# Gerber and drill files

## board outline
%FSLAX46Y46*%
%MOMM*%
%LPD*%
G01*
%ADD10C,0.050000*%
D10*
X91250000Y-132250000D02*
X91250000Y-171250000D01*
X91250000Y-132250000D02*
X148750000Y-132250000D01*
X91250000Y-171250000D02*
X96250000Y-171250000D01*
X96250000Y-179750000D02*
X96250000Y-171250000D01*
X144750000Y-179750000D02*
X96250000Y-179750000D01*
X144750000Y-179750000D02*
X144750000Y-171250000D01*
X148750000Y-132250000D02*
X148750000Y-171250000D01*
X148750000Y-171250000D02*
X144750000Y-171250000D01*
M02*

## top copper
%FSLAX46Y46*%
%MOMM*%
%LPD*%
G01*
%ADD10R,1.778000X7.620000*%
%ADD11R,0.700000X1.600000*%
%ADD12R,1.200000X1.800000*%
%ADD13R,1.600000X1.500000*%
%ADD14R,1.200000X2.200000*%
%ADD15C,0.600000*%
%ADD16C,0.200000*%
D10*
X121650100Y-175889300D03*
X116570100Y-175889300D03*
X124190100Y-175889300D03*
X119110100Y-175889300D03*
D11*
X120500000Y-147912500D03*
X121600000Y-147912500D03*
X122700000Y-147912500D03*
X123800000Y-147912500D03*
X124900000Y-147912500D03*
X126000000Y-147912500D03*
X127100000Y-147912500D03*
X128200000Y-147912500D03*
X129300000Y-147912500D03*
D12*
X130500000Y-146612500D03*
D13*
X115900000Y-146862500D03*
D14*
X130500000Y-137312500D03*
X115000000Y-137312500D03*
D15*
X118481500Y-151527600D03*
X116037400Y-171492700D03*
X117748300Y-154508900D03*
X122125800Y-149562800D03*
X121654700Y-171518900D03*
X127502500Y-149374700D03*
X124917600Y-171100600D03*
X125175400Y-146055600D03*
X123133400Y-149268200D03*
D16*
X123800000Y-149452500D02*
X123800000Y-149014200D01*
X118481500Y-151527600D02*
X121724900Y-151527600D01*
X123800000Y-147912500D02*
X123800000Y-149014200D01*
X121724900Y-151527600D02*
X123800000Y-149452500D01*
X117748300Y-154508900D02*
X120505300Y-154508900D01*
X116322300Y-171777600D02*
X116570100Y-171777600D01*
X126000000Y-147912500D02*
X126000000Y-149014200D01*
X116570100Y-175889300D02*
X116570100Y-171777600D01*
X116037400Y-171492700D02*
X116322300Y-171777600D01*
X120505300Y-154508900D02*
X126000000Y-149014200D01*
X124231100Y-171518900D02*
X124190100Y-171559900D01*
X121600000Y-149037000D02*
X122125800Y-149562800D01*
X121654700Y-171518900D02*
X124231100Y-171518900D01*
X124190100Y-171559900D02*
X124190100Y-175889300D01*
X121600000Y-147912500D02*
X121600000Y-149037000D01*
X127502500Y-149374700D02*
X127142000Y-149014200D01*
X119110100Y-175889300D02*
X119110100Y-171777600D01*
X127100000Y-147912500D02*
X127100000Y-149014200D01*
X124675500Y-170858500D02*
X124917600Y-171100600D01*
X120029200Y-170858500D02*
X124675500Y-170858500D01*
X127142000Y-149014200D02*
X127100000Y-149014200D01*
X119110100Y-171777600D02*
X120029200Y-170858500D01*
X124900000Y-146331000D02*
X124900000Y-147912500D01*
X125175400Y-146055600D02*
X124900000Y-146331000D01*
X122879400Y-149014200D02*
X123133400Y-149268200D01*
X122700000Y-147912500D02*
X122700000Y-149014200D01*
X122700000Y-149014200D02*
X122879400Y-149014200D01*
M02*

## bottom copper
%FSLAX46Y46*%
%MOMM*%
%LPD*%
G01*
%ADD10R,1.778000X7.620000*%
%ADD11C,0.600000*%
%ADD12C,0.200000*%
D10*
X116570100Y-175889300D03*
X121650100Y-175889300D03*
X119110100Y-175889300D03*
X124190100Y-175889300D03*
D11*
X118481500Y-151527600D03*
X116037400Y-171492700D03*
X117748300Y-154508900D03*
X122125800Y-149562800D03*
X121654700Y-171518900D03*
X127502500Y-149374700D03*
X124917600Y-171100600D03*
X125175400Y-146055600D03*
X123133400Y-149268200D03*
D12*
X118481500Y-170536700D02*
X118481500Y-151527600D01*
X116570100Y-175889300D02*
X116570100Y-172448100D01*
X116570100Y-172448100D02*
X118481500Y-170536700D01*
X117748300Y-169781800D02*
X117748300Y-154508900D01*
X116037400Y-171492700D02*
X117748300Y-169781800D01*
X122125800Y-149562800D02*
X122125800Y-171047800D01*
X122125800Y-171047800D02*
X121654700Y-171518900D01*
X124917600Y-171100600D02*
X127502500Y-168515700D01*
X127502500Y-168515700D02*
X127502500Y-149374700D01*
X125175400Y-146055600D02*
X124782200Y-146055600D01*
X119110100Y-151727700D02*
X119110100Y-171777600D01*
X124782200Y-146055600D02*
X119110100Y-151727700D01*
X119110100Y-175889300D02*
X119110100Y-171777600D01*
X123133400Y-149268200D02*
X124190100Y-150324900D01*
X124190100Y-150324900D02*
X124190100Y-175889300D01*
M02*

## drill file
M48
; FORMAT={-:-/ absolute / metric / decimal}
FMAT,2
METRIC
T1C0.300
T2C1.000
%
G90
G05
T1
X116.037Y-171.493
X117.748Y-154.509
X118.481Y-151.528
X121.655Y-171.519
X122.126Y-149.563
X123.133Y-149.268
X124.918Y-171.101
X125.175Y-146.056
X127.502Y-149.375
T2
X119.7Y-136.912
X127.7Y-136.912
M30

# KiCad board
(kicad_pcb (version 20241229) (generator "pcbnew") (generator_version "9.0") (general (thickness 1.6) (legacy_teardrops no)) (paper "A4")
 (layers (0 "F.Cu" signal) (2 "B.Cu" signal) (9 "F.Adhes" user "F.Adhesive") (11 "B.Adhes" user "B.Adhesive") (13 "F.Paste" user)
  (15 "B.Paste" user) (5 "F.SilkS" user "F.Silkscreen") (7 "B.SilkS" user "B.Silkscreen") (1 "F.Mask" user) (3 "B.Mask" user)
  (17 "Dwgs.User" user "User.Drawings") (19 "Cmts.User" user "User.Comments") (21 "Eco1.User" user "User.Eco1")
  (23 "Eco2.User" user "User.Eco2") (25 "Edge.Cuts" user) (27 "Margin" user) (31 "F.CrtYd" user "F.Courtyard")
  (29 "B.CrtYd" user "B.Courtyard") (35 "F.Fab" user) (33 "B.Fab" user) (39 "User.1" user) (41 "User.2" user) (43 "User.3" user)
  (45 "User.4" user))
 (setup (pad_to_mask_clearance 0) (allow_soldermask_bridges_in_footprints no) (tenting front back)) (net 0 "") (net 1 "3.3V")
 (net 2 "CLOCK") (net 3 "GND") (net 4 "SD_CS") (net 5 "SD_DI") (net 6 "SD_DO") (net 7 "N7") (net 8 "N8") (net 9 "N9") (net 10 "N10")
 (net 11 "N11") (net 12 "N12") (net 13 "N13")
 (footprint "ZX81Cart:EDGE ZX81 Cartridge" (layer "F.Cu") (at 119.7451 172.7143)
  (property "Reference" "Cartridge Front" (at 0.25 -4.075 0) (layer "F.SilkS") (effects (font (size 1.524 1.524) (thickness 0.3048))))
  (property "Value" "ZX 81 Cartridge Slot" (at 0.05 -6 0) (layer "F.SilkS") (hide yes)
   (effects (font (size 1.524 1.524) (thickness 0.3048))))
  (pad "3.3V" connect rect (at -3.175 3.175 180) (size 1.778 7.62) (layers "B.Cu" "B.Mask") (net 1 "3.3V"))
  (pad "A3" connect rect (at 1.905 3.175 180) (size 1.778 7.62) (layers "F.Cu" "F.Mask"))
  (pad "B3" connect rect (at 1.905 3.175 180) (size 1.778 7.62) (layers "B.Cu" "B.Mask"))
  (pad "CLOCK" connect rect (at -0.635 3.175 180) (size 1.778 7.62) (layers "B.Cu" "B.Mask") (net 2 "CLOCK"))
  (pad "GND" connect rect (at -3.175 3.175 180) (size 1.778 7.62) (layers "F.Cu" "F.Mask") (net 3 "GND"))
  (pad "SD_CS" connect rect (at 4.445 3.175 180) (size 1.778 7.62) (layers "F.Cu" "F.Mask") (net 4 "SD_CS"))
  (pad "SD_DI" connect rect (at -0.635 3.175 180) (size 1.778 7.62) (layers "F.Cu" "F.Mask") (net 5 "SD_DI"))
  (pad "SD_DO" connect rect (at 4.445 3.175 180) (size 1.778 7.62) (layers "B.Cu" "B.Mask") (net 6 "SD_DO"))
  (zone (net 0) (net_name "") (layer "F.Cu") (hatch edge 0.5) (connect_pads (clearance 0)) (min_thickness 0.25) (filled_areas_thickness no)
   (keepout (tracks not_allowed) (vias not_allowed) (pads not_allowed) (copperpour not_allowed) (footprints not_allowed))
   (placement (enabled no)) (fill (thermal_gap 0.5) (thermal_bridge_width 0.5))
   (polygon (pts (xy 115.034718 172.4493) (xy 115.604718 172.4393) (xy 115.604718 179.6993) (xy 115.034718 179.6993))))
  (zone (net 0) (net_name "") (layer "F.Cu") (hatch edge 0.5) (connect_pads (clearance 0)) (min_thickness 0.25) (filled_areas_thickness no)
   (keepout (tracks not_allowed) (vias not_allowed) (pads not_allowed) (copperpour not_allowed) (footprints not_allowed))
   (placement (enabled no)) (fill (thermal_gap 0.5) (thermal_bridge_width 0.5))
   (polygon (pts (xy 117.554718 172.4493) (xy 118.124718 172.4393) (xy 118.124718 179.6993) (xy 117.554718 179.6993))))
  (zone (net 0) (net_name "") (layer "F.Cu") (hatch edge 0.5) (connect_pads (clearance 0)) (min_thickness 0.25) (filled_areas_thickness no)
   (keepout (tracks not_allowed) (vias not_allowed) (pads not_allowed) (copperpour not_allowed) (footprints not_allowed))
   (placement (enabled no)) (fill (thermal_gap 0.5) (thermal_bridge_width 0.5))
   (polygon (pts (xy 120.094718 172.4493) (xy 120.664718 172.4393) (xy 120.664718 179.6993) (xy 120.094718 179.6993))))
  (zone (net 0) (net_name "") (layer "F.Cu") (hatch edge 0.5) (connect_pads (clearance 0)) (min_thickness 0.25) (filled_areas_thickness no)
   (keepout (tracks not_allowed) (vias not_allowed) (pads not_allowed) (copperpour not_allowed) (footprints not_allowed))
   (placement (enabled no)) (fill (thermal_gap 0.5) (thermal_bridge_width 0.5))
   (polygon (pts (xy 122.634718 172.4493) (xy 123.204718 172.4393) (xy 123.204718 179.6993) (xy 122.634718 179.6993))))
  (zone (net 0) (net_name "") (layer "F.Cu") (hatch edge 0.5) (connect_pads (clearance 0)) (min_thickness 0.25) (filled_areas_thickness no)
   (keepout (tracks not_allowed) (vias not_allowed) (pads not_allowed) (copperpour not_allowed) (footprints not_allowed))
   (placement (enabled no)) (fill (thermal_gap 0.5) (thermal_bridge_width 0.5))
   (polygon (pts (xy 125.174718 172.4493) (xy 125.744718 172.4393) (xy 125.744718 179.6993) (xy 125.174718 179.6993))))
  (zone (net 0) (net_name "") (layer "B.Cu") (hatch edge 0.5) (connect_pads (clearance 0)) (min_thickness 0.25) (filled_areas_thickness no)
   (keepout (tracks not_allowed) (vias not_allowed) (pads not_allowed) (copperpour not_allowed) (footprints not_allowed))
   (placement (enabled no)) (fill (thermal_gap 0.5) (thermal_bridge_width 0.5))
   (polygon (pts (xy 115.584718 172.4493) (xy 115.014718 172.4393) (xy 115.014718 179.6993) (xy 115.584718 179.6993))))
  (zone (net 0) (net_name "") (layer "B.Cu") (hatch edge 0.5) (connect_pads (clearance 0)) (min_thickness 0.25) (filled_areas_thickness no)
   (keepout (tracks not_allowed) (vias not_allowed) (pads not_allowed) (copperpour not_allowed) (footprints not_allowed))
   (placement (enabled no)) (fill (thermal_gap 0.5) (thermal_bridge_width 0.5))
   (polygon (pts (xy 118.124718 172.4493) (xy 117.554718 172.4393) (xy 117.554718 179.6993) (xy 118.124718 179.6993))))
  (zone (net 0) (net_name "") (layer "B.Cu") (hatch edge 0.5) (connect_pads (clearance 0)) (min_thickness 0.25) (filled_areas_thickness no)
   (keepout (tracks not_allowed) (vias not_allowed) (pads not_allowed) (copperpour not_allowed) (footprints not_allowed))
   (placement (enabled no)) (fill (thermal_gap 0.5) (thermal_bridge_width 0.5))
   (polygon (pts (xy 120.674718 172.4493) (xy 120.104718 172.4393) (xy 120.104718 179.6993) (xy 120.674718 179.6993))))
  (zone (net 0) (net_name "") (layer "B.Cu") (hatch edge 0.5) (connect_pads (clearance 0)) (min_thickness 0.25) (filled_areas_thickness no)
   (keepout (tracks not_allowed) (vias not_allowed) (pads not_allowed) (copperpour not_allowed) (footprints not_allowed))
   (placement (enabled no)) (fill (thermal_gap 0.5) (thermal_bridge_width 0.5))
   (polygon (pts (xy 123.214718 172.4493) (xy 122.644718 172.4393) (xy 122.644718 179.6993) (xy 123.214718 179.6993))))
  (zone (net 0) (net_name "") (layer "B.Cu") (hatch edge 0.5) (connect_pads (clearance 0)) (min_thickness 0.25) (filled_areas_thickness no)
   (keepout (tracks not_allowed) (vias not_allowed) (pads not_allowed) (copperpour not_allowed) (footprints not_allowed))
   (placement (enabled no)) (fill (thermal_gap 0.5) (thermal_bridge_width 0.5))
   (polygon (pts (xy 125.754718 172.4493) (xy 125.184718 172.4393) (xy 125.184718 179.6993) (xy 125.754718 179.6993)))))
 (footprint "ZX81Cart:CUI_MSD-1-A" (layer "F.Cu") (at 122.75 140.1625 180)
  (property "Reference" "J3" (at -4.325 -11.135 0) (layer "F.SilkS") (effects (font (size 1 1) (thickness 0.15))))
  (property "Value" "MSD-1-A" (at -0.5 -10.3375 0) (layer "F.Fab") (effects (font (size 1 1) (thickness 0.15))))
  (pad "" np_thru_hole circle (at -4.95 3.25 180) (size 1 1) (drill 1) (layers "*.Cu" "*.Mask"))
  (pad "" np_thru_hole circle (at 3.05 3.25 180) (size 1 1) (drill 1) (layers "*.Cu" "*.Mask"))
  (pad "1" smd rect (at 2.25 -7.75 180) (size 0.7 1.6) (layers "F.Cu" "F.Mask" "F.Paste") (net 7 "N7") (solder_mask_margin 0.102))
  (pad "2" smd rect (at 1.15 -7.75 180) (size 0.7 1.6) (layers "F.Cu" "F.Mask" "F.Paste") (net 4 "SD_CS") (solder_mask_margin 0.102))
  (pad "3" smd rect (at 0.05 -7.75 180) (size 0.7 1.6) (layers "F.Cu" "F.Mask" "F.Paste") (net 6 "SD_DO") (solder_mask_margin 0.102))
  (pad "4" smd rect (at -1.05 -7.75 180) (size 0.7 1.6) (layers "F.Cu" "F.Mask" "F.Paste") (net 1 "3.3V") (solder_mask_margin 0.102))
  (pad "5" smd rect (at -2.15 -7.75 180) (size 0.7 1.6) (layers "F.Cu" "F.Mask" "F.Paste") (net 2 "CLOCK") (solder_mask_margin 0.102))
  (pad "6" smd rect (at -3.25 -7.75 180) (size 0.7 1.6) (layers "F.Cu" "F.Mask" "F.Paste") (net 3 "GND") (solder_mask_margin 0.102))
  (pad "7" smd rect (at -4.35 -7.75 180) (size 0.7 1.6) (layers "F.Cu" "F.Mask" "F.Paste") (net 5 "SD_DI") (solder_mask_margin 0.102))
  (pad "8" smd rect (at -5.45 -7.75 180) (size 0.7 1.6) (layers "F.Cu" "F.Mask" "F.Paste") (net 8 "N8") (solder_mask_margin 0.102))
  (pad "CD" smd rect (at -6.55 -7.75 180) (size 0.7 1.6) (layers "F.Cu" "F.Mask" "F.Paste") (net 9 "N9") (solder_mask_margin 0.102))
  (pad "G1" smd rect (at -7.75 -6.45 180) (size 1.2 1.8) (layers "F.Cu" "F.Mask" "F.Paste") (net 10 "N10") (solder_mask_margin 0.102))
  (pad "G2" smd rect (at 6.85 -6.7 180) (size 1.6 1.5) (layers "F.Cu" "F.Mask" "F.Paste") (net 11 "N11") (solder_mask_margin 0.102))
  (pad "G3" smd rect (at -7.75 2.85 180) (size 1.2 2.2) (layers "F.Cu" "F.Mask" "F.Paste") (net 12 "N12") (solder_mask_margin 0.102))
  (pad "G4" smd rect (at 7.75 2.85 180) (size 1.2 2.2) (layers "F.Cu" "F.Mask" "F.Paste") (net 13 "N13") (solder_mask_margin 0.102)))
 (gr_line (start 91.25 132.25) (end 91.25 171.25) (stroke (width 0.05) (type default)) (layer "Edge.Cuts"))
 (gr_line (start 91.25 132.25) (end 148.75 132.25) (stroke (width 0.05) (type default)) (layer "Edge.Cuts"))
 (gr_line (start 91.25 171.25) (end 96.25 171.25) (stroke (width 0.05) (type default)) (layer "Edge.Cuts"))
 (gr_line (start 96.25 179.75) (end 96.25 171.25) (stroke (width 0.05) (type default)) (layer "Edge.Cuts"))
 (gr_line (start 144.75 179.75) (end 96.25 179.75) (stroke (width 0.05) (type solid)) (layer "Edge.Cuts"))
 (gr_line (start 144.75 179.75) (end 144.75 171.25) (stroke (width 0.05) (type default)) (layer "Edge.Cuts"))
 (gr_line (start 148.75 132.25) (end 148.75 171.25) (stroke (width 0.05) (type default)) (layer "Edge.Cuts"))
 (gr_line (start 148.75 171.25) (end 144.75 171.25) (stroke (width 0.05) (type default)) (layer "Edge.Cuts"))
 (segment (start 123.8 149.4525) (end 123.8 149.0142) (width 0.2) (layer "F.Cu") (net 1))
 (segment (start 118.4815 151.5276) (end 121.7249 151.5276) (width 0.2) (layer "F.Cu") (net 1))
 (segment (start 123.8 147.9125) (end 123.8 149.0142) (width 0.2) (layer "F.Cu") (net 1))
 (segment (start 121.7249 151.5276) (end 123.8 149.4525) (width 0.2) (layer "F.Cu") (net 1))
 (via (at 118.4815 151.5276) (size 0.6) (drill 0.3) (layers "F.Cu" "B.Cu") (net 1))
 (segment (start 118.4815 170.5367) (end 118.4815 151.5276) (width 0.2) (layer "B.Cu") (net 1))
 (segment (start 116.5701 175.8893) (end 116.5701 172.4481) (width 0.2) (layer "B.Cu") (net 1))
 (segment (start 116.5701 172.4481) (end 118.4815 170.5367) (width 0.2) (layer "B.Cu") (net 1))
 (segment (start 117.7483 154.5089) (end 120.5053 154.5089) (width 0.2) (layer "F.Cu") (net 3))
 (segment (start 116.3223 171.7776) (end 116.5701 171.7776) (width 0.2) (layer "F.Cu") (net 3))
 (segment (start 126 147.9125) (end 126 149.0142) (width 0.2) (layer "F.Cu") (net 3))
 (segment (start 116.5701 175.8893) (end 116.5701 171.7776) (width 0.2) (layer "F.Cu") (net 3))
 (segment (start 116.0374 171.4927) (end 116.3223 171.7776) (width 0.2) (layer "F.Cu") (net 3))
 (segment (start 120.5053 154.5089) (end 126 149.0142) (width 0.2) (layer "F.Cu") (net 3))
 (via (at 116.0374 171.4927) (size 0.6) (drill 0.3) (layers "F.Cu" "B.Cu") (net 3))
 (via (at 117.7483 154.5089) (size 0.6) (drill 0.3) (layers "F.Cu" "B.Cu") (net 3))
 (segment (start 117.7483 169.7818) (end 117.7483 154.5089) (width 0.2) (layer "B.Cu") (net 3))
 (segment (start 116.0374 171.4927) (end 117.7483 169.7818) (width 0.2) (layer "B.Cu") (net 3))
 (segment (start 124.2311 171.5189) (end 124.1901 171.5599) (width 0.2) (layer "F.Cu") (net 4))
 (segment (start 121.6 149.037) (end 122.1258 149.5628) (width 0.2) (layer "F.Cu") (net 4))
 (segment (start 121.6547 171.5189) (end 124.2311 171.5189) (width 0.2) (layer "F.Cu") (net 4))
 (segment (start 124.1901 171.5599) (end 124.1901 175.8893) (width 0.2) (layer "F.Cu") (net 4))
 (segment (start 121.6 147.9125) (end 121.6 149.037) (width 0.2) (layer "F.Cu") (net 4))
 (via (at 122.1258 149.5628) (size 0.6) (drill 0.3) (layers "F.Cu" "B.Cu") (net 4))
 (via (at 121.6547 171.5189) (size 0.6) (drill 0.3) (layers "F.Cu" "B.Cu") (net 4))
 (segment (start 122.1258 149.5628) (end 122.1258 171.0478) (width 0.2) (layer "B.Cu") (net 4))
 (segment (start 122.1258 171.0478) (end 121.6547 171.5189) (width 0.2) (layer "B.Cu") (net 4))
 (segment (start 127.5025 149.3747) (end 127.142 149.0142) (width 0.2) (layer "F.Cu") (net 5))
 (segment (start 119.1101 175.8893) (end 119.1101 171.7776) (width 0.2) (layer "F.Cu") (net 5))
 (segment (start 127.1 147.9125) (end 127.1 149.0142) (width 0.2) (layer "F.Cu") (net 5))
 (segment (start 124.6755 170.8585) (end 124.9176 171.1006) (width 0.2) (layer "F.Cu") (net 5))
 (segment (start 120.0292 170.8585) (end 124.6755 170.8585) (width 0.2) (layer "F.Cu") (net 5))
 (segment (start 127.142 149.0142) (end 127.1 149.0142) (width 0.2) (layer "F.Cu") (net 5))
 (segment (start 119.1101 171.7776) (end 120.0292 170.8585) (width 0.2) (layer "F.Cu") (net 5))
 (via (at 127.5025 149.3747) (size 0.6) (drill 0.3) (layers "F.Cu" "B.Cu") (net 5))
 (via (at 124.9176 171.1006) (size 0.6) (drill 0.3) (layers "F.Cu" "B.Cu") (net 5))
 (segment (start 124.9176 171.1006) (end 127.5025 168.5157) (width 0.2) (layer "B.Cu") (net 5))
 (segment (start 127.5025 168.5157) (end 127.5025 149.3747) (width 0.2) (layer "B.Cu") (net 5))
 (segment (start 124.9 146.331) (end 124.9 147.9125) (width 0.2) (layer "F.Cu") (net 2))
 (segment (start 125.1754 146.0556) (end 124.9 146.331) (width 0.2) (layer "F.Cu") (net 2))
 (via (at 125.1754 146.0556) (size 0.6) (drill 0.3) (layers "F.Cu" "B.Cu") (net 2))
 (segment (start 125.1754 146.0556) (end 124.7822 146.0556) (width 0.2) (layer "B.Cu") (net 2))
 (segment (start 119.1101 151.7277) (end 119.1101 171.7776) (width 0.2) (layer "B.Cu") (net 2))
 (segment (start 124.7822 146.0556) (end 119.1101 151.7277) (width 0.2) (layer "B.Cu") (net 2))
 (segment (start 119.1101 175.8893) (end 119.1101 171.7776) (width 0.2) (layer "B.Cu") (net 2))
 (segment (start 122.8794 149.0142) (end 123.1334 149.2682) (width 0.2) (layer "F.Cu") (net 6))
 (segment (start 122.7 147.9125) (end 122.7 149.0142) (width 0.2) (layer "F.Cu") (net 6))
 (segment (start 122.7 149.0142) (end 122.8794 149.0142) (width 0.2) (layer "F.Cu") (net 6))
 (via (at 123.1334 149.2682) (size 0.6) (drill 0.3) (layers "F.Cu" "B.Cu") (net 6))
 (segment (start 123.1334 149.2682) (end 124.1901 150.3249) (width 0.2) (layer "B.Cu") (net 6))
 (segment (start 124.1901 150.3249) (end 124.1901 175.8893) (width 0.2) (layer "B.Cu") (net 6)))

